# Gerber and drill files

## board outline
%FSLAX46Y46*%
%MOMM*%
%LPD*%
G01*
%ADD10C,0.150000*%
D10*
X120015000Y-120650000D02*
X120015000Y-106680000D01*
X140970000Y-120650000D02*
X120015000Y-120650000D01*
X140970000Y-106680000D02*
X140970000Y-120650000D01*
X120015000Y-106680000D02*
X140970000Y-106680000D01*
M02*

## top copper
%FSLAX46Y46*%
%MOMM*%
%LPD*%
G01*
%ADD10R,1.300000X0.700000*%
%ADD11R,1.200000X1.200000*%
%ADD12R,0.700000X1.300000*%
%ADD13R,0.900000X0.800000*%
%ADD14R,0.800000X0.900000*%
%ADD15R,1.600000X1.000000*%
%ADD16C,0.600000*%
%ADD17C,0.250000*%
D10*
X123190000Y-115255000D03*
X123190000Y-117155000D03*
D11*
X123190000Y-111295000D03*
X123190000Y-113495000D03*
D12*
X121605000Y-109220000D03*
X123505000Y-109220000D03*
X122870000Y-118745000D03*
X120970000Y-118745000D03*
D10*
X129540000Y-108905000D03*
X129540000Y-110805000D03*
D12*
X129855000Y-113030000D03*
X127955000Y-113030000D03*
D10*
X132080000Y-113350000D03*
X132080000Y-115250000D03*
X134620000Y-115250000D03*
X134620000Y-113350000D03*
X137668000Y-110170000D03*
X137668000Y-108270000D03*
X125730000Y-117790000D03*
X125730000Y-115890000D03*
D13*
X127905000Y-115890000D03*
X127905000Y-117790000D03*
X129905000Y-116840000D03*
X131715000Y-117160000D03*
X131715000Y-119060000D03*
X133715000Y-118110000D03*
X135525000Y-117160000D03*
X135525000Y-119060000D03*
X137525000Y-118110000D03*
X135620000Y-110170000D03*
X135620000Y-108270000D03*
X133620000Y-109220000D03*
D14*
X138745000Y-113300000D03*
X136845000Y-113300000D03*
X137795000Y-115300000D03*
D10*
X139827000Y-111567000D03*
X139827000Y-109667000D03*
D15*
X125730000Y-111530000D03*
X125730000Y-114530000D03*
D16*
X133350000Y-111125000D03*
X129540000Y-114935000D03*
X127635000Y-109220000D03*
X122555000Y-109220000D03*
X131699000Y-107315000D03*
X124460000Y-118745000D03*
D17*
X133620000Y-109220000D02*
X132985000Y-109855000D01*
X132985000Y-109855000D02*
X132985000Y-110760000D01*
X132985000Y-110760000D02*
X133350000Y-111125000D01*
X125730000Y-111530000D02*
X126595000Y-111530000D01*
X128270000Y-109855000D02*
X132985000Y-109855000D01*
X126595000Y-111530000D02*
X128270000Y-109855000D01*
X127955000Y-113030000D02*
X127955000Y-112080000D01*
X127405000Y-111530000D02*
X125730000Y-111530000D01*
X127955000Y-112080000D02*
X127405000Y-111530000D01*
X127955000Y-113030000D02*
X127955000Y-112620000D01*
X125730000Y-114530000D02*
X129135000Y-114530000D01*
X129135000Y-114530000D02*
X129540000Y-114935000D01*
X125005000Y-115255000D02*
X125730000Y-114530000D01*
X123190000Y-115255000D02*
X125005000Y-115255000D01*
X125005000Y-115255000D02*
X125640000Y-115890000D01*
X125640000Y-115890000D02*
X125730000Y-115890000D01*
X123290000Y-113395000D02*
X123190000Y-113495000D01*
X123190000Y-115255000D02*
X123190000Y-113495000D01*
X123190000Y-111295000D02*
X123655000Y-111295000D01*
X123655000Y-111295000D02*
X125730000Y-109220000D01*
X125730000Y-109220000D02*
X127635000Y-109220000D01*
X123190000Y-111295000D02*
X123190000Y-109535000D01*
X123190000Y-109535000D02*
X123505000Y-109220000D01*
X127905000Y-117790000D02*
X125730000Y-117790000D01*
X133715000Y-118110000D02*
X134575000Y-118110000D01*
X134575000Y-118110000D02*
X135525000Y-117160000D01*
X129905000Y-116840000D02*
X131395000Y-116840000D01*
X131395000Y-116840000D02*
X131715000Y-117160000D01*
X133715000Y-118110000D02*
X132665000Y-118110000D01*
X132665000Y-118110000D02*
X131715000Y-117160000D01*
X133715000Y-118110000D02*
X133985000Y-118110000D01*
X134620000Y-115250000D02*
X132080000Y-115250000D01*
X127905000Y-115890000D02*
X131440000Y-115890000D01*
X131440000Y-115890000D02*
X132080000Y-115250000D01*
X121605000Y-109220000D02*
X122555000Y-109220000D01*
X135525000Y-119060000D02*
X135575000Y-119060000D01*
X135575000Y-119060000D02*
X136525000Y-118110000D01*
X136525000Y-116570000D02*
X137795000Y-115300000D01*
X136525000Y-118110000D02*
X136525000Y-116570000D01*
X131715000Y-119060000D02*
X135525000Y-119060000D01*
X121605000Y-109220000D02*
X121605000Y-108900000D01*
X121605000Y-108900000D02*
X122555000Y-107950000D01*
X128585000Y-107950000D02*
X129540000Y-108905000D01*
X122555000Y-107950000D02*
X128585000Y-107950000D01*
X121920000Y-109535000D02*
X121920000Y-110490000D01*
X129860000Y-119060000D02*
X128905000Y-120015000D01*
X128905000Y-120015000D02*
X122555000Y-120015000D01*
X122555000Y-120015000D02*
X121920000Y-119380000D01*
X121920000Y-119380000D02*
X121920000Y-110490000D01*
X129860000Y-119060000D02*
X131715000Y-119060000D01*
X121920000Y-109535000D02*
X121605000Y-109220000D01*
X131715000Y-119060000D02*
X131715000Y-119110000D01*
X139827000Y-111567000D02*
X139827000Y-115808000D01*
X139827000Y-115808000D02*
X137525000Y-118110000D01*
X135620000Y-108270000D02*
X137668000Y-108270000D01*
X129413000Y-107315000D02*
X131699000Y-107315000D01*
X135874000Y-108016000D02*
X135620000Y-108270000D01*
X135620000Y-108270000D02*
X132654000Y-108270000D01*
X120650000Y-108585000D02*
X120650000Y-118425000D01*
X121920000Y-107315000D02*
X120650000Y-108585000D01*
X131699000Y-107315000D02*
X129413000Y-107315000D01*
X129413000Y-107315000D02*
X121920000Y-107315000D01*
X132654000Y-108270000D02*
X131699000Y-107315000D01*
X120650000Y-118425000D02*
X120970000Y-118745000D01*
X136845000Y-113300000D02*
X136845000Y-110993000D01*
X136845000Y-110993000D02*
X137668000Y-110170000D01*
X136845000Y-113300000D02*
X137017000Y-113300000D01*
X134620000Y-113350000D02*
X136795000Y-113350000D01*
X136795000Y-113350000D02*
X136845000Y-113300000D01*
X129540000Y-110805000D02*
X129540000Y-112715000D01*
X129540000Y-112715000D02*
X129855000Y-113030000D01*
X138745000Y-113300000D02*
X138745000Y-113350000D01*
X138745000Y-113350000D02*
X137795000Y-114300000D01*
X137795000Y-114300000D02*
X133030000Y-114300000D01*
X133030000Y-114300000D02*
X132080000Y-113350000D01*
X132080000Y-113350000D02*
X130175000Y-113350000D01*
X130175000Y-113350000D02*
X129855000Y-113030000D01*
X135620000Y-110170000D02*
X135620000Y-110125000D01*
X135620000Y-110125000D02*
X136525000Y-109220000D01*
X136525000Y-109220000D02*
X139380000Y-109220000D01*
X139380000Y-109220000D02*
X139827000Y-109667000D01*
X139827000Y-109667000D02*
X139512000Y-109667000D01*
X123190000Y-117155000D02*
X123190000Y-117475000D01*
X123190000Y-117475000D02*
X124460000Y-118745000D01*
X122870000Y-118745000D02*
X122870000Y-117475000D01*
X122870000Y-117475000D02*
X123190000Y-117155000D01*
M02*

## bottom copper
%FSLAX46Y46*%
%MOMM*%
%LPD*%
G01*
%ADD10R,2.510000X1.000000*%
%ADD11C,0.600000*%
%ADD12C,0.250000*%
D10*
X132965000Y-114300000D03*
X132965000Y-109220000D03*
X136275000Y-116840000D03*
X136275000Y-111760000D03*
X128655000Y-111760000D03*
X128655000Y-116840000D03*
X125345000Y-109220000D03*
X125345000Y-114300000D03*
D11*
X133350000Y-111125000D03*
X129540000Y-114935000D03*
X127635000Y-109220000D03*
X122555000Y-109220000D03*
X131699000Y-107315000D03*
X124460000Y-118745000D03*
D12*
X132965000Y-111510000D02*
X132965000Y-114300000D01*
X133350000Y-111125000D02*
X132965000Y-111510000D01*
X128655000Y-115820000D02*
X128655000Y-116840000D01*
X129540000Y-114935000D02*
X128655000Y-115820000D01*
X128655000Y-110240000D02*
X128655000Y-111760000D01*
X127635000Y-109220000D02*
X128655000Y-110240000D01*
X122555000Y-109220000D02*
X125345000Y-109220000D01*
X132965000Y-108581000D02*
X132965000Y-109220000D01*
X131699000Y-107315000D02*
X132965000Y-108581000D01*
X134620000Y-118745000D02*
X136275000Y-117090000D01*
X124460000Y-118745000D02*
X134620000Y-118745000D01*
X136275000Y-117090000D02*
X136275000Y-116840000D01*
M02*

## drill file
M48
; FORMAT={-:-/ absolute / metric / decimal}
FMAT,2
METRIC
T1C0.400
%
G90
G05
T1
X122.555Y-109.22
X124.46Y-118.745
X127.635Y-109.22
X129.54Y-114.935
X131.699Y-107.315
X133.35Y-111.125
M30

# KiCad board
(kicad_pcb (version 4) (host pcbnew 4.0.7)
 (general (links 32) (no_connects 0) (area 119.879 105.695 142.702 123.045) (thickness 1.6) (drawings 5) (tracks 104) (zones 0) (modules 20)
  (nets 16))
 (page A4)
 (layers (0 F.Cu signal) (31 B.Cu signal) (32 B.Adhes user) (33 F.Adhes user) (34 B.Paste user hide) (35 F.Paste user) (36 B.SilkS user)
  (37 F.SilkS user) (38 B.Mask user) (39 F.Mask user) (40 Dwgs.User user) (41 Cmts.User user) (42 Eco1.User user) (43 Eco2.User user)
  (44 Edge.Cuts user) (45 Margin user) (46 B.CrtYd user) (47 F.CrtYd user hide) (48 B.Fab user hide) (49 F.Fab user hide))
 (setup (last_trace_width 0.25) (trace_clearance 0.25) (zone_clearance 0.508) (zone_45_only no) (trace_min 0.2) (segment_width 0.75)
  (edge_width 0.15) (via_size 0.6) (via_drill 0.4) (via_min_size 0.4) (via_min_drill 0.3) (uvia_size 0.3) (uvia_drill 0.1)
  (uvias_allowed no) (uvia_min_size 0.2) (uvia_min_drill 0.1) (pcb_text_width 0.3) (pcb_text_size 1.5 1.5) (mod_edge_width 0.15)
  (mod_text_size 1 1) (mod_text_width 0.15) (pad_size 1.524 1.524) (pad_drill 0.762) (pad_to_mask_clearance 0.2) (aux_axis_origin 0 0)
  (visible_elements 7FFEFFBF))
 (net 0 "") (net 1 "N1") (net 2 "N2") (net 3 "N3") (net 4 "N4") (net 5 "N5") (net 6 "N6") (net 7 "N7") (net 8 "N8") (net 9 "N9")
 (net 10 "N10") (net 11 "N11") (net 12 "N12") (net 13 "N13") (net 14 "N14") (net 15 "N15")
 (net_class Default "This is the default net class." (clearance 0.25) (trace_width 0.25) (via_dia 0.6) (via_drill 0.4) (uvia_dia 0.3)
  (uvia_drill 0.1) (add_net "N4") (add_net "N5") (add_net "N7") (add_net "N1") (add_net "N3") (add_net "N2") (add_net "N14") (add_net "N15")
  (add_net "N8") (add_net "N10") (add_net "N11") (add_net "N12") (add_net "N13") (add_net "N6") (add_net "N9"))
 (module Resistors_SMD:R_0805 (layer F.Cu) (at 123.19 116.205 270)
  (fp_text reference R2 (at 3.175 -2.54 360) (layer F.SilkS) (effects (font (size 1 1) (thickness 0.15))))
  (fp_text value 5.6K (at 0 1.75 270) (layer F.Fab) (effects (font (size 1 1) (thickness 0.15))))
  (pad 1 smd rect (at -0.95 0 270) (size 0.7 1.3) (layers F.Cu F.Paste F.Mask) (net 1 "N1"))
  (pad 2 smd rect (at 0.95 0 270) (size 0.7 1.3) (layers F.Cu F.Paste F.Mask) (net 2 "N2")))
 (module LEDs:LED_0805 (layer F.Cu) (at 123.19 112.395 90)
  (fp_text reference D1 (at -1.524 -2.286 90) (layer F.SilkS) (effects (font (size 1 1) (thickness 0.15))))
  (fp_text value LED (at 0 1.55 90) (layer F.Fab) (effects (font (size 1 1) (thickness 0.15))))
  (pad 2 smd rect (at 1.1 0 270) (size 1.2 1.2) (layers F.Cu F.Paste F.Mask) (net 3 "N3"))
  (pad 1 smd rect (at -1.1 0 270) (size 1.2 1.2) (layers F.Cu F.Paste F.Mask) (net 1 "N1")))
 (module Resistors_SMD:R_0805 (layer F.Cu) (at 122.555 109.22)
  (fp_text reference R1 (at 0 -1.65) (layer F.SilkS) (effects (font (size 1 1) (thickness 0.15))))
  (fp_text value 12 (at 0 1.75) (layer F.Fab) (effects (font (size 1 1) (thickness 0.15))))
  (pad 1 smd rect (at -0.95 0) (size 0.7 1.3) (layers F.Cu F.Paste F.Mask) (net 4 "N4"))
  (pad 2 smd rect (at 0.95 0) (size 0.7 1.3) (layers F.Cu F.Paste F.Mask) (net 3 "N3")))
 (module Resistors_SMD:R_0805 (layer F.Cu) (at 121.92 118.745 180)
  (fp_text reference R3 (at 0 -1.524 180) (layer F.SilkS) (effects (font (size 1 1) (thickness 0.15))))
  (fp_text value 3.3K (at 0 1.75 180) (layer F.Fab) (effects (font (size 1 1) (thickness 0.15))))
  (pad 1 smd rect (at -0.95 0 180) (size 0.7 1.3) (layers F.Cu F.Paste F.Mask) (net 2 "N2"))
  (pad 2 smd rect (at 0.95 0 180) (size 0.7 1.3) (layers F.Cu F.Paste F.Mask) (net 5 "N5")))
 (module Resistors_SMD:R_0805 (layer F.Cu) (at 129.54 109.855 270)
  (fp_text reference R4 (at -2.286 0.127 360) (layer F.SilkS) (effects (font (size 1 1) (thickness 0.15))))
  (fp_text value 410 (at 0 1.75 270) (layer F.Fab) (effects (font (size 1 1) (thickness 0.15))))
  (pad 1 smd rect (at -0.95 0 270) (size 0.7 1.3) (layers F.Cu F.Paste F.Mask) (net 4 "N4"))
  (pad 2 smd rect (at 0.95 0 270) (size 0.7 1.3) (layers F.Cu F.Paste F.Mask) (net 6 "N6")))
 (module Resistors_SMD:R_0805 (layer F.Cu) (at 128.905 113.03 180)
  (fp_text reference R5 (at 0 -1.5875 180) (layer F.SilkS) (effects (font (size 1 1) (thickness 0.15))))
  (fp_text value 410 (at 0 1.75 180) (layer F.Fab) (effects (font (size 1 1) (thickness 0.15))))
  (pad 1 smd rect (at -0.95 0 180) (size 0.7 1.3) (layers F.Cu F.Paste F.Mask) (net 6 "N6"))
  (pad 2 smd rect (at 0.95 0 180) (size 0.7 1.3) (layers F.Cu F.Paste F.Mask) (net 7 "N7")))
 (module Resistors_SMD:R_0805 (layer F.Cu) (at 132.08 114.3 270)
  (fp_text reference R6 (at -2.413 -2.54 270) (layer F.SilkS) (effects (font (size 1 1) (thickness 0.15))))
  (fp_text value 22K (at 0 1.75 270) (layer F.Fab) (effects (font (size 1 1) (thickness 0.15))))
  (pad 1 smd rect (at -0.95 0 270) (size 0.7 1.3) (layers F.Cu F.Paste F.Mask) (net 6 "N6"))
  (pad 2 smd rect (at 0.95 0 270) (size 0.7 1.3) (layers F.Cu F.Paste F.Mask) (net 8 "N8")))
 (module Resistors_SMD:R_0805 (layer F.Cu) (at 134.62 114.3 90)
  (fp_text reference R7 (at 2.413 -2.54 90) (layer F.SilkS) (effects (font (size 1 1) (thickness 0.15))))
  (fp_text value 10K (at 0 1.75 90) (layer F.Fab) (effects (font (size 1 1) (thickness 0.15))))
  (pad 1 smd rect (at -0.95 0 90) (size 0.7 1.3) (layers F.Cu F.Paste F.Mask) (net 8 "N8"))
  (pad 2 smd rect (at 0.95 0 90) (size 0.7 1.3) (layers F.Cu F.Paste F.Mask) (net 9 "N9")))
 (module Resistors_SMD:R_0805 (layer F.Cu) (at 137.668 109.22 90)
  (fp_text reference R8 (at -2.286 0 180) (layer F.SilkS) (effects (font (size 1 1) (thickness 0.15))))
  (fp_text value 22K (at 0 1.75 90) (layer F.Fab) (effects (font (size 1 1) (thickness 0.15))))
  (pad 1 smd rect (at -0.95 0 90) (size 0.7 1.3) (layers F.Cu F.Paste F.Mask) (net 9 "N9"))
  (pad 2 smd rect (at 0.95 0 90) (size 0.7 1.3) (layers F.Cu F.Paste F.Mask) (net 5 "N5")))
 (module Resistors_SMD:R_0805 (layer F.Cu) (at 125.73 116.84 90)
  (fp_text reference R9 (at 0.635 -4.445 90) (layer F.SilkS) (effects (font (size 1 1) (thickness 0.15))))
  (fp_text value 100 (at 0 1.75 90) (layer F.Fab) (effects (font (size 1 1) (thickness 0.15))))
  (pad 1 smd rect (at -0.95 0 90) (size 0.7 1.3) (layers F.Cu F.Paste F.Mask) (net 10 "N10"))
  (pad 2 smd rect (at 0.95 0 90) (size 0.7 1.3) (layers F.Cu F.Paste F.Mask) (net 1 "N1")))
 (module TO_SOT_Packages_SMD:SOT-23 (layer F.Cu) (at 128.905 116.84)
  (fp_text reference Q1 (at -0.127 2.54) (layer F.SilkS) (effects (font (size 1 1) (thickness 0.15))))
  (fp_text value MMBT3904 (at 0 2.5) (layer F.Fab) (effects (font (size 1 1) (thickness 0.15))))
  (pad 1 smd rect (at -1 -0.95) (size 0.9 0.8) (layers F.Cu F.Paste F.Mask) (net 8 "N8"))
  (pad 2 smd rect (at -1 0.95) (size 0.9 0.8) (layers F.Cu F.Paste F.Mask) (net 10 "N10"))
  (pad 3 smd rect (at 1 0) (size 0.9 0.8) (layers F.Cu F.Paste F.Mask) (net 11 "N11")))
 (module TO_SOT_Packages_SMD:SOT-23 (layer F.Cu) (at 132.715 118.11)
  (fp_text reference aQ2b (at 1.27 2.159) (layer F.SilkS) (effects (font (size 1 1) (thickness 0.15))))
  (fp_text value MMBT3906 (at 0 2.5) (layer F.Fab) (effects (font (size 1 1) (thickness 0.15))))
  (pad 1 smd rect (at -1 -0.95) (size 0.9 0.8) (layers F.Cu F.Paste F.Mask) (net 11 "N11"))
  (pad 2 smd rect (at -1 0.95) (size 0.9 0.8) (layers F.Cu F.Paste F.Mask) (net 4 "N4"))
  (pad 3 smd rect (at 1 0) (size 0.9 0.8) (layers F.Cu F.Paste F.Mask) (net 11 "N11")))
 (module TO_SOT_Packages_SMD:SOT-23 (layer F.Cu) (at 136.525 118.11)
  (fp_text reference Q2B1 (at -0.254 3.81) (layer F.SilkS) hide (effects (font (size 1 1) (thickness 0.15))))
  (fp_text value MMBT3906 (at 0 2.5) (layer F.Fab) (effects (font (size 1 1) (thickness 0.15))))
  (pad 1 smd rect (at -1 -0.95) (size 0.9 0.8) (layers F.Cu F.Paste F.Mask) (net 11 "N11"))
  (pad 2 smd rect (at -1 0.95) (size 0.9 0.8) (layers F.Cu F.Paste F.Mask) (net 4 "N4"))
  (pad 3 smd rect (at 1 0) (size 0.9 0.8) (layers F.Cu F.Paste F.Mask) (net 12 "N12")))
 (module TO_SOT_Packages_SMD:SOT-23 (layer F.Cu) (at 134.62 109.22 180)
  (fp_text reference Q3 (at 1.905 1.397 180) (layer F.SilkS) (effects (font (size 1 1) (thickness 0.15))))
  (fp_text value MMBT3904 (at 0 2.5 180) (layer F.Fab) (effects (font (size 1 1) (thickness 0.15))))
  (pad 1 smd rect (at -1 -0.95 180) (size 0.9 0.8) (layers F.Cu F.Paste F.Mask) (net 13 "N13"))
  (pad 2 smd rect (at -1 0.95 180) (size 0.9 0.8) (layers F.Cu F.Paste F.Mask) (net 5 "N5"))
  (pad 3 smd rect (at 1 0 180) (size 0.9 0.8) (layers F.Cu F.Paste F.Mask) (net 7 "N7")))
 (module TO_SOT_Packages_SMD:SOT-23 (layer F.Cu) (at 137.795 114.3 270)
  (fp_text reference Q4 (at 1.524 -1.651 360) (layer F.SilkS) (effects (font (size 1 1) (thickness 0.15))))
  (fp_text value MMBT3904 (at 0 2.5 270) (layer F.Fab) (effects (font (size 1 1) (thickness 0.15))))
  (pad 1 smd rect (at -1 -0.95 270) (size 0.9 0.8) (layers F.Cu F.Paste F.Mask) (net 6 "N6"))
  (pad 2 smd rect (at -1 0.95 270) (size 0.9 0.8) (layers F.Cu F.Paste F.Mask) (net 9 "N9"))
  (pad 3 smd rect (at 1 0 270) (size 0.9 0.8) (layers F.Cu F.Paste F.Mask) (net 4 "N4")))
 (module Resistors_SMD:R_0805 (layer F.Cu) (at 139.827 110.617 90)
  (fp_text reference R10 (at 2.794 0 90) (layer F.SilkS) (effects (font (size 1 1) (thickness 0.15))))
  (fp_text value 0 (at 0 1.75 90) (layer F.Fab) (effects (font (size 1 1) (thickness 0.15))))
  (pad 1 smd rect (at -0.95 0 90) (size 0.7 1.3) (layers F.Cu F.Paste F.Mask) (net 12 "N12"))
  (pad 2 smd rect (at 0.95 0 90) (size 0.7 1.3) (layers F.Cu F.Paste F.Mask) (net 13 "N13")))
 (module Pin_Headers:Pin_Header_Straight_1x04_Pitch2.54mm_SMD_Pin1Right (layer B.Cu) (at 134.62 113.03)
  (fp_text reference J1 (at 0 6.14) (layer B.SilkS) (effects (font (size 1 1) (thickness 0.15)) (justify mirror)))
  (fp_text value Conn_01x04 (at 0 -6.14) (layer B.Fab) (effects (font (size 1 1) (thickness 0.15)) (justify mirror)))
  (pad 2 smd rect (at -1.655 1.27) (size 2.51 1) (layers B.Cu B.Paste B.Mask) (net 7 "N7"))
  (pad 4 smd rect (at -1.655 -3.81) (size 2.51 1) (layers B.Cu B.Paste B.Mask) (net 5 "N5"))
  (pad 1 smd rect (at 1.655 3.81) (size 2.51 1) (layers B.Cu B.Paste B.Mask) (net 2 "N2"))
  (pad 3 smd rect (at 1.655 -1.27) (size 2.51 1) (layers B.Cu B.Paste B.Mask) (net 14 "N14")))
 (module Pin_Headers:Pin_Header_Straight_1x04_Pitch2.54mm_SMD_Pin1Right (layer B.Cu) (at 127 113.03 180)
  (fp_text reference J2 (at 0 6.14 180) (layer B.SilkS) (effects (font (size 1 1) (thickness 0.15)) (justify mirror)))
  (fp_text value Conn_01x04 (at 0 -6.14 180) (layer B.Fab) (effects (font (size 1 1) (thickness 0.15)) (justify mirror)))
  (pad 2 smd rect (at -1.655 1.27 180) (size 2.51 1) (layers B.Cu B.Paste B.Mask) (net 3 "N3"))
  (pad 4 smd rect (at -1.655 -3.81 180) (size 2.51 1) (layers B.Cu B.Paste B.Mask) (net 1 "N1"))
  (pad 1 smd rect (at 1.655 3.81 180) (size 2.51 1) (layers B.Cu B.Paste B.Mask) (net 4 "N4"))
  (pad 3 smd rect (at 1.655 -1.27 180) (size 2.51 1) (layers B.Cu B.Paste B.Mask) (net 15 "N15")))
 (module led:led (layer F.Cu) (at 123.571 112.776 270)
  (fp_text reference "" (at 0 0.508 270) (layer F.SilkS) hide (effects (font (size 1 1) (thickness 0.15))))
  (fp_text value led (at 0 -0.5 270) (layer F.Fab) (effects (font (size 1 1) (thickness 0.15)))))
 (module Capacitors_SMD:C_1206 (layer F.Cu) (at 125.73 113.03 270)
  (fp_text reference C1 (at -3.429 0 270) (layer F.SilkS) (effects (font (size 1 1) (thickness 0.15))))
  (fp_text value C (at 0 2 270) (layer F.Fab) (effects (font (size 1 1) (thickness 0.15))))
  (pad 1 smd rect (at -1.5 0 270) (size 1 1.6) (layers F.Cu F.Paste F.Mask) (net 7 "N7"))
  (pad 2 smd rect (at 1.5 0 270) (size 1 1.6) (layers F.Cu F.Paste F.Mask) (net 1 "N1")))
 (gr_line (start 120.015 120.65) (end 120.015 106.68) (angle 90) (layer Edge.Cuts) (width 0.15))
 (gr_line (start 140.97 120.65) (end 120.015 120.65) (angle 90) (layer Edge.Cuts) (width 0.15))
 (gr_line (start 140.97 106.68) (end 140.97 120.65) (angle 90) (layer Edge.Cuts) (width 0.15))
 (gr_line (start 120.015 106.68) (end 140.97 106.68) (angle 90) (layer Edge.Cuts) (width 0.15))
 (segment (start 133.62 109.22) (end 132.985 109.855) (width 0.25) (layer F.Cu) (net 7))
 (segment (start 132.985 109.855) (end 132.985 110.76) (width 0.25) (layer F.Cu) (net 7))
 (segment (start 132.965 111.51) (end 132.965 114.3) (width 0.25) (layer B.Cu) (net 7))
 (segment (start 133.35 111.125) (end 132.965 111.51) (width 0.25) (layer B.Cu) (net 7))
 (via (at 133.35 111.125) (size 0.6) (drill 0.4) (layers F.Cu B.Cu) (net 7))
 (segment (start 132.985 110.76) (end 133.35 111.125) (width 0.25) (layer F.Cu) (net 7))
 (segment (start 125.73 111.53) (end 126.595 111.53) (width 0.25) (layer F.Cu) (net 7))
 (segment (start 128.27 109.855) (end 132.985 109.855) (width 0.25) (layer F.Cu) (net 7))
 (segment (start 126.595 111.53) (end 128.27 109.855) (width 0.25) (layer F.Cu) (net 7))
 (segment (start 127.955 113.03) (end 127.955 112.08) (width 0.25) (layer F.Cu) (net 7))
 (segment (start 127.405 111.53) (end 125.73 111.53) (width 0.25) (layer F.Cu) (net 7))
 (segment (start 127.955 112.08) (end 127.405 111.53) (width 0.25) (layer F.Cu) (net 7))
 (segment (start 127.955 113.03) (end 127.955 112.62) (width 0.25) (layer F.Cu) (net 7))
 (segment (start 125.73 114.53) (end 129.135 114.53) (width 0.25) (layer F.Cu) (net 1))
 (segment (start 128.655 115.82) (end 128.655 116.84) (width 0.25) (layer B.Cu) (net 1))
 (segment (start 129.54 114.935) (end 128.655 115.82) (width 0.25) (layer B.Cu) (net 1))
 (via (at 129.54 114.935) (size 0.6) (drill 0.4) (layers F.Cu B.Cu) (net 1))
 (segment (start 129.135 114.53) (end 129.54 114.935) (width 0.25) (layer F.Cu) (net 1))
 (segment (start 125.005 115.255) (end 125.73 114.53) (width 0.25) (layer F.Cu) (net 1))
 (segment (start 123.19 115.255) (end 125.005 115.255) (width 0.25) (layer F.Cu) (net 1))
 (segment (start 125.005 115.255) (end 125.64 115.89) (width 0.25) (layer F.Cu) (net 1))
 (segment (start 125.64 115.89) (end 125.73 115.89) (width 0.25) (layer F.Cu) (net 1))
 (segment (start 123.29 113.395) (end 123.19 113.495) (width 0.25) (layer F.Cu) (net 1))
 (segment (start 123.19 115.255) (end 123.19 113.495) (width 0.25) (layer F.Cu) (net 1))
 (segment (start 123.19 111.295) (end 123.655 111.295) (width 0.25) (layer F.Cu) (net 3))
 (segment (start 123.655 111.295) (end 125.73 109.22) (width 0.25) (layer F.Cu) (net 3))
 (segment (start 128.655 110.24) (end 128.655 111.76) (width 0.25) (layer B.Cu) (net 3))
 (segment (start 127.635 109.22) (end 128.655 110.24) (width 0.25) (layer B.Cu) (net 3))
 (via (at 127.635 109.22) (size 0.6) (drill 0.4) (layers F.Cu B.Cu) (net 3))
 (segment (start 125.73 109.22) (end 127.635 109.22) (width 0.25) (layer F.Cu) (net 3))
 (segment (start 123.19 111.295) (end 123.19 109.535) (width 0.25) (layer F.Cu) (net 3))
 (segment (start 123.19 109.535) (end 123.505 109.22) (width 0.25) (layer F.Cu) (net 3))
 (segment (start 127.905 117.79) (end 125.73 117.79) (width 0.25) (layer F.Cu) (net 10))
 (segment (start 133.715 118.11) (end 134.575 118.11) (width 0.25) (layer F.Cu) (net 11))
 (segment (start 134.575 118.11) (end 135.525 117.16) (width 0.25) (layer F.Cu) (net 11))
 (segment (start 129.905 116.84) (end 131.395 116.84) (width 0.25) (layer F.Cu) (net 11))
 (segment (start 131.395 116.84) (end 131.715 117.16) (width 0.25) (layer F.Cu) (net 11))
 (segment (start 133.715 118.11) (end 132.665 118.11) (width 0.25) (layer F.Cu) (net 11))
 (segment (start 132.665 118.11) (end 131.715 117.16) (width 0.25) (layer F.Cu) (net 11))
 (segment (start 133.715 118.11) (end 133.985 118.11) (width 0.25) (layer F.Cu) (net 11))
 (segment (start 134.62 115.25) (end 132.08 115.25) (width 0.25) (layer F.Cu) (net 8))
 (segment (start 127.905 115.89) (end 131.44 115.89) (width 0.25) (layer F.Cu) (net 8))
 (segment (start 131.44 115.89) (end 132.08 115.25) (width 0.25) (layer F.Cu) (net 8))
 (segment (start 121.605 109.22) (end 122.555 109.22) (width 0.25) (layer F.Cu) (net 4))
 (segment (start 122.555 109.22) (end 125.345 109.22) (width 0.25) (layer B.Cu) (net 4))
 (via (at 122.555 109.22) (size 0.6) (drill 0.4) (layers F.Cu B.Cu) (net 4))
 (segment (start 135.525 119.06) (end 135.575 119.06) (width 0.25) (layer F.Cu) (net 4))
 (segment (start 135.575 119.06) (end 136.525 118.11) (width 0.25) (layer F.Cu) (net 4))
 (segment (start 136.525 116.57) (end 137.795 115.3) (width 0.25) (layer F.Cu) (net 4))
 (segment (start 136.525 118.11) (end 136.525 116.57) (width 0.25) (layer F.Cu) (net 4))
 (segment (start 131.715 119.06) (end 135.525 119.06) (width 0.25) (layer F.Cu) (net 4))
 (segment (start 121.605 109.22) (end 121.605 108.9) (width 0.25) (layer F.Cu) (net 4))
 (segment (start 121.605 108.9) (end 122.555 107.95) (width 0.25) (layer F.Cu) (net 4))
 (segment (start 128.585 107.95) (end 129.54 108.905) (width 0.25) (layer F.Cu) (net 4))
 (segment (start 122.555 107.95) (end 128.585 107.95) (width 0.25) (layer F.Cu) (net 4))
 (segment (start 121.92 109.535) (end 121.92 110.49) (width 0.25) (layer F.Cu) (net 4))
 (segment (start 129.86 119.06) (end 128.905 120.015) (width 0.25) (layer F.Cu) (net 4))
 (segment (start 128.905 120.015) (end 122.555 120.015) (width 0.25) (layer F.Cu) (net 4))
 (segment (start 122.555 120.015) (end 121.92 119.38) (width 0.25) (layer F.Cu) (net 4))
 (segment (start 121.92 119.38) (end 121.92 110.49) (width 0.25) (layer F.Cu) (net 4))
 (segment (start 129.86 119.06) (end 131.715 119.06) (width 0.25) (layer F.Cu) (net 4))
 (segment (start 121.92 109.535) (end 121.605 109.22) (width 0.25) (layer F.Cu) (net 4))
 (segment (start 131.715 119.06) (end 131.715 119.11) (width 0.25) (layer F.Cu) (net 4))
 (segment (start 139.827 111.567) (end 139.827 115.808) (width 0.25) (layer F.Cu) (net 12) (status 400000))
 (segment (start 139.827 115.808) (end 137.525 118.11) (width 0.25) (layer F.Cu) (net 12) (status 800000))
 (segment (start 135.62 108.27) (end 137.668 108.27) (width 0.25) (layer F.Cu) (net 5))
 (segment (start 129.413 107.315) (end 131.699 107.315) (width 0.25) (layer F.Cu) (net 5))
 (segment (start 132.965 108.581) (end 132.965 109.22) (width 0.25) (layer B.Cu) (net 5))
 (segment (start 131.699 107.315) (end 132.965 108.581) (width 0.25) (layer B.Cu) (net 5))
 (via (at 131.699 107.315) (size 0.6) (drill 0.4) (layers F.Cu B.Cu) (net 5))
 (segment (start 135.874 108.016) (end 135.62 108.27) (width 0.25) (layer F.Cu) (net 5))
 (segment (start 135.62 108.27) (end 132.654 108.27) (width 0.25) (layer F.Cu) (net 5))
 (segment (start 120.65 108.585) (end 120.65 118.425) (width 0.25) (layer F.Cu) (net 5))
 (segment (start 121.92 107.315) (end 120.65 108.585) (width 0.25) (layer F.Cu) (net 5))
 (segment (start 131.699 107.315) (end 129.413 107.315) (width 0.25) (layer F.Cu) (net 5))
 (segment (start 129.413 107.315) (end 121.92 107.315) (width 0.25) (layer F.Cu) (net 5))
 (segment (start 132.654 108.27) (end 131.699 107.315) (width 0.25) (layer F.Cu) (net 5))
 (segment (start 120.65 118.425) (end 120.97 118.745) (width 0.25) (layer F.Cu) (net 5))
 (segment (start 136.845 113.3) (end 136.845 110.993) (width 0.25) (layer F.Cu) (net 9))
 (segment (start 136.845 110.993) (end 137.668 110.17) (width 0.25) (layer F.Cu) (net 9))
 (segment (start 136.845 113.3) (end 137.017 113.3) (width 0.25) (layer F.Cu) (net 9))
 (segment (start 134.62 113.35) (end 136.795 113.35) (width 0.25) (layer F.Cu) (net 9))
 (segment (start 136.795 113.35) (end 136.845 113.3) (width 0.25) (layer F.Cu) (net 9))
 (segment (start 129.54 110.805) (end 129.54 112.715) (width 0.25) (layer F.Cu) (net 6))
 (segment (start 129.54 112.715) (end 129.855 113.03) (width 0.25) (layer F.Cu) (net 6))
 (segment (start 138.745 113.3) (end 138.745 113.35) (width 0.25) (layer F.Cu) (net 6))
 (segment (start 138.745 113.35) (end 137.795 114.3) (width 0.25) (layer F.Cu) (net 6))
 (segment (start 137.795 114.3) (end 133.03 114.3) (width 0.25) (layer F.Cu) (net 6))
 (segment (start 133.03 114.3) (end 132.08 113.35) (width 0.25) (layer F.Cu) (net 6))
 (segment (start 132.08 113.35) (end 130.175 113.35) (width 0.25) (layer F.Cu) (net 6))
 (segment (start 130.175 113.35) (end 129.855 113.03) (width 0.25) (layer F.Cu) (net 6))
 (segment (start 135.62 110.17) (end 135.62 110.125) (width 0.25) (layer F.Cu) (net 13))
 (segment (start 135.62 110.125) (end 136.525 109.22) (width 0.25) (layer F.Cu) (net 13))
 (segment (start 136.525 109.22) (end 139.38 109.22) (width 0.25) (layer F.Cu) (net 13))
 (segment (start 139.38 109.22) (end 139.827 109.667) (width 0.25) (layer F.Cu) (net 13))
 (segment (start 139.827 109.667) (end 139.512 109.667) (width 0.25) (layer F.Cu) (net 13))
 (segment (start 123.19 117.155) (end 123.19 117.475) (width 0.25) (layer F.Cu) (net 2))
 (segment (start 123.19 117.475) (end 124.46 118.745) (width 0.25) (layer F.Cu) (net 2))
 (segment (start 134.62 118.745) (end 136.275 117.09) (width 0.25) (layer B.Cu) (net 2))
 (segment (start 124.46 118.745) (end 134.62 118.745) (width 0.25) (layer B.Cu) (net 2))
 (via (at 124.46 118.745) (size 0.6) (drill 0.4) (layers F.Cu B.Cu) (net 2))
 (segment (start 136.275 117.09) (end 136.275 116.84) (width 0.25) (layer B.Cu) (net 2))
 (segment (start 122.87 118.745) (end 122.87 117.475) (width 0.25) (layer F.Cu) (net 2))
 (segment (start 122.87 117.475) (end 123.19 117.155) (width 0.25) (layer F.Cu) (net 2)))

